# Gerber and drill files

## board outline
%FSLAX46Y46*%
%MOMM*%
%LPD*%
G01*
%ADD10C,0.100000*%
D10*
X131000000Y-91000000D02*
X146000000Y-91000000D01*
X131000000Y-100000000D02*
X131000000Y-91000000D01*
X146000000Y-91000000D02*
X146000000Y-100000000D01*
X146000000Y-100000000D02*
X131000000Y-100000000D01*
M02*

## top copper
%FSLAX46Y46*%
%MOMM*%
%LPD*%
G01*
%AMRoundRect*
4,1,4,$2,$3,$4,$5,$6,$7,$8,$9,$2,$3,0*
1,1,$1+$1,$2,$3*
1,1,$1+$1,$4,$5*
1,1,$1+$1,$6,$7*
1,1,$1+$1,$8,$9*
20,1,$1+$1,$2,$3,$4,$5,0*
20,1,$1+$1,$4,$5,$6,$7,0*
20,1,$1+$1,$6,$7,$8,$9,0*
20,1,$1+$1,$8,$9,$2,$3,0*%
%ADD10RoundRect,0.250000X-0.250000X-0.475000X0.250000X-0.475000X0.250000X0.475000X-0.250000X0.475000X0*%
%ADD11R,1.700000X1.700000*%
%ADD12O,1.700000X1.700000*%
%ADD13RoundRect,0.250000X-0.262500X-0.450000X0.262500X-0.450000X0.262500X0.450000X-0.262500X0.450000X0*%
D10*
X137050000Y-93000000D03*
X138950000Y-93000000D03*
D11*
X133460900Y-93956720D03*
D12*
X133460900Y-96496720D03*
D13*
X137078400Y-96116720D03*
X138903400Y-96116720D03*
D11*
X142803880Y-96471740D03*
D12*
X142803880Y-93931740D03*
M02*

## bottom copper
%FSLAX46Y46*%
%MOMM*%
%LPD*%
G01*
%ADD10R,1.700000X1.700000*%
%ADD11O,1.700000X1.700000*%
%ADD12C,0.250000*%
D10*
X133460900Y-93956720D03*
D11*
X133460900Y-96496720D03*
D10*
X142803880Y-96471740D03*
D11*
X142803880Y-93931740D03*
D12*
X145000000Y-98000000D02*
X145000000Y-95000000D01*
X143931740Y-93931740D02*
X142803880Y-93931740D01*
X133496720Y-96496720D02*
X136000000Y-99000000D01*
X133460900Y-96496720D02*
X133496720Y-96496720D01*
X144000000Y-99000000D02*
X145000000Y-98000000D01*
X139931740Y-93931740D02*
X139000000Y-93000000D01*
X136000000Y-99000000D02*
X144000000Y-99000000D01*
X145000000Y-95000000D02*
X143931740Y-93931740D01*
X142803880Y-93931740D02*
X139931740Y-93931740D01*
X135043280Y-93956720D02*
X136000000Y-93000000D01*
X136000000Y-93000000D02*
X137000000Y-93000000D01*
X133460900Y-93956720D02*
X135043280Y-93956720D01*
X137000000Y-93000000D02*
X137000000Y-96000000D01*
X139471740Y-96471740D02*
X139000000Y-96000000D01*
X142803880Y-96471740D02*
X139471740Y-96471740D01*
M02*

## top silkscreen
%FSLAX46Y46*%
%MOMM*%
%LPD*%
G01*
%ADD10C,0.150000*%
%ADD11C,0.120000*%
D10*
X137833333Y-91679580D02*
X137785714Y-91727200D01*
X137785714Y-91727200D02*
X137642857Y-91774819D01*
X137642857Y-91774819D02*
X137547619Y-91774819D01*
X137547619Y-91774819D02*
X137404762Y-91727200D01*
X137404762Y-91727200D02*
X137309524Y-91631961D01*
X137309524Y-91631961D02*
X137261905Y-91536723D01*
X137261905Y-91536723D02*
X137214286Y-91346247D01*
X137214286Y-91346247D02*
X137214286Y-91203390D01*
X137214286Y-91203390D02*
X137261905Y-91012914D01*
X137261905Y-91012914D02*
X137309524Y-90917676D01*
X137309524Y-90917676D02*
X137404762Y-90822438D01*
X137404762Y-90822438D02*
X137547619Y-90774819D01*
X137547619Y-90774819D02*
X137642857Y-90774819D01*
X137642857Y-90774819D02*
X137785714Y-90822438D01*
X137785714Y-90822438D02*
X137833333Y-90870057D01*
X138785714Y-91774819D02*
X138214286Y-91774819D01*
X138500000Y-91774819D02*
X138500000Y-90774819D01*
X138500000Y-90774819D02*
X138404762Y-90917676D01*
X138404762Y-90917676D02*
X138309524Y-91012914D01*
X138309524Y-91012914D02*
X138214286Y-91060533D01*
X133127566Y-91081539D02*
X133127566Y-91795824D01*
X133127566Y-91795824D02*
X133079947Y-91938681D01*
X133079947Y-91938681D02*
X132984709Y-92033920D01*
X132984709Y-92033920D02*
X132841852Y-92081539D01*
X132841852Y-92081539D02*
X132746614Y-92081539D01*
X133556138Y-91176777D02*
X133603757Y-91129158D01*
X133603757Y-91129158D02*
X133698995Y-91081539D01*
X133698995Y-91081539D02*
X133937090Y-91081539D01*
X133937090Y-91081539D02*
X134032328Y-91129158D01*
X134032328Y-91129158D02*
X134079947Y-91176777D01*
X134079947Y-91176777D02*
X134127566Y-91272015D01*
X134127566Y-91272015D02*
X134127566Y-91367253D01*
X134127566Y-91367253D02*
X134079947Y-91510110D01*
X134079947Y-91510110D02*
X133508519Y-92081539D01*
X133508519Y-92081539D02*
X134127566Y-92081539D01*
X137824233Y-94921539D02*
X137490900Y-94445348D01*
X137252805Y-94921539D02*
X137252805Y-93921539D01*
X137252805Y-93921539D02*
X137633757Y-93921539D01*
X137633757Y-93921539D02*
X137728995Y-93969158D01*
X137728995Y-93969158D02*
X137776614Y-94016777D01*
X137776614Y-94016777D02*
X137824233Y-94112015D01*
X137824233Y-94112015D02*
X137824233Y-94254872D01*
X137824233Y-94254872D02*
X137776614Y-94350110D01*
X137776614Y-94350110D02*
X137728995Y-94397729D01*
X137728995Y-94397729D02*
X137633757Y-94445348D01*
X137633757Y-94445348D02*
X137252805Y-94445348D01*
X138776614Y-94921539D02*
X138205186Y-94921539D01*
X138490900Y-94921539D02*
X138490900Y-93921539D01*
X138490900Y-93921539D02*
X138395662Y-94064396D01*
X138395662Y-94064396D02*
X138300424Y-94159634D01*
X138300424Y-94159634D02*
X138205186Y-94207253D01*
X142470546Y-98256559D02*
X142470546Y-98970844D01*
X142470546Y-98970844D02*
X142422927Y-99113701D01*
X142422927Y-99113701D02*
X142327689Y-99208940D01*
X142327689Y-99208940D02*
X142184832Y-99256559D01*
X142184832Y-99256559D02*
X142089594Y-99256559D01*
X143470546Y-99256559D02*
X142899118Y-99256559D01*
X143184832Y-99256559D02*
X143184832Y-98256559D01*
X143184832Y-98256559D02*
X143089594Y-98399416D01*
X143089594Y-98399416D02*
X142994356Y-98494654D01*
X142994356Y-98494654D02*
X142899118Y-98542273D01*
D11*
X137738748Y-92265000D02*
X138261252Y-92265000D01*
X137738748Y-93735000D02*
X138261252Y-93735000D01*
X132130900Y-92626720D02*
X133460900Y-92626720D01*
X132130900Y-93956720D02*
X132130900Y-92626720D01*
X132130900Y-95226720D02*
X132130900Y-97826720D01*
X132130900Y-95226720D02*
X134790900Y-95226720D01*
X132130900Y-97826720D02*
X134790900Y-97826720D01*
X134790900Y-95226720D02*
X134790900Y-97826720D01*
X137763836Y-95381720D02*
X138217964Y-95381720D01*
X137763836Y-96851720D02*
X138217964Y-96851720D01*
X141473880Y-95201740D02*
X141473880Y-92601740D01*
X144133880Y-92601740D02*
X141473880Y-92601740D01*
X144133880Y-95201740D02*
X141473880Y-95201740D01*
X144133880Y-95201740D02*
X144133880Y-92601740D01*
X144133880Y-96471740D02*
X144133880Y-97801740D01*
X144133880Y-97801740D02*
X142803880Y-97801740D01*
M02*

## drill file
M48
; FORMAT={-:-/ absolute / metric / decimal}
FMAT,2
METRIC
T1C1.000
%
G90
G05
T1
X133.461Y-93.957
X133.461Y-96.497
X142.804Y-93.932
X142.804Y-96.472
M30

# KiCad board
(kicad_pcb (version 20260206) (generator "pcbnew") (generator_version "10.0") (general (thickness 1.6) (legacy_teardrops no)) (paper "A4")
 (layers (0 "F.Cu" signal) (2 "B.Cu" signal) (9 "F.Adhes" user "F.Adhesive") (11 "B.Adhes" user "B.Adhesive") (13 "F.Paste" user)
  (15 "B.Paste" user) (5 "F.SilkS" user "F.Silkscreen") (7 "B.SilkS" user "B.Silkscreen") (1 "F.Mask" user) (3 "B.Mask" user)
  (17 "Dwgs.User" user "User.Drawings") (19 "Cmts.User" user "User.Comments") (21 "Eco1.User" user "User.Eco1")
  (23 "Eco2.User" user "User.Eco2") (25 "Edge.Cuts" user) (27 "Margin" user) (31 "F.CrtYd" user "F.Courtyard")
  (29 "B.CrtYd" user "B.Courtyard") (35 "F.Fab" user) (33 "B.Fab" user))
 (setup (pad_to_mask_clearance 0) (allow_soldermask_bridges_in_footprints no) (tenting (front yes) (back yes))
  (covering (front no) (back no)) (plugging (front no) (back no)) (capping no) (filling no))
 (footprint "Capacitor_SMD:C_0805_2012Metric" (layer "F.Cu") (at 138 93)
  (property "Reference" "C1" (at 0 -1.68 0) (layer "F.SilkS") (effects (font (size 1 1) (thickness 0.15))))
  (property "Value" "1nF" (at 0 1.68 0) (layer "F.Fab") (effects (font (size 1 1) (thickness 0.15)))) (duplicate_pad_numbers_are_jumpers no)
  (fp_line (start -0.261252 -0.735) (end 0.261252 -0.735) (stroke (width 0.12) (type solid)) (layer "F.SilkS"))
  (fp_line (start -0.261252 0.735) (end 0.261252 0.735) (stroke (width 0.12) (type solid)) (layer "F.SilkS"))
  (pad "1" smd roundrect (at -0.95 0) (size 1 1.45) (layers "F.Cu" "F.Mask" "F.Paste") (roundrect_rratio 0.25) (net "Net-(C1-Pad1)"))
  (pad "2" smd roundrect (at 0.95 0) (size 1 1.45) (layers "F.Cu" "F.Mask" "F.Paste") (roundrect_rratio 0.25) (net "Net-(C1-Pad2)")))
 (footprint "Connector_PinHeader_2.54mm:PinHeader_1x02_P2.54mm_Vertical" (layer "F.Cu") (at 133.4609 93.95672)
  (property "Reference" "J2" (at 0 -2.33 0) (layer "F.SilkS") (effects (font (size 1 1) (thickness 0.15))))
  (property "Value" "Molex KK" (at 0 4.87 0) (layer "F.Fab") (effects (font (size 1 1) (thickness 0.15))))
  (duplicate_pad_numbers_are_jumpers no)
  (fp_line (start -1.33 -1.33) (end 0 -1.33) (stroke (width 0.12) (type solid)) (layer "F.SilkS"))
  (fp_line (start -1.33 0) (end -1.33 -1.33) (stroke (width 0.12) (type solid)) (layer "F.SilkS"))
  (fp_line (start -1.33 1.27) (end -1.33 3.87) (stroke (width 0.12) (type solid)) (layer "F.SilkS"))
  (fp_line (start -1.33 1.27) (end 1.33 1.27) (stroke (width 0.12) (type solid)) (layer "F.SilkS"))
  (fp_line (start -1.33 3.87) (end 1.33 3.87) (stroke (width 0.12) (type solid)) (layer "F.SilkS"))
  (fp_line (start 1.33 1.27) (end 1.33 3.87) (stroke (width 0.12) (type solid)) (layer "F.SilkS"))
  (pad "1" thru_hole rect (at 0 0) (size 1.7 1.7) (drill 1) (layers "*.Cu" "*.Mask") (remove_unused_layers no) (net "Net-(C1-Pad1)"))
  (pad "2" thru_hole oval (at 0 2.54) (size 1.7 1.7) (drill 1) (layers "*.Cu" "*.Mask") (remove_unused_layers no) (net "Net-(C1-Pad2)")))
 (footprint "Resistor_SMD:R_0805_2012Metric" (layer "F.Cu") (at 137.9909 96.11672)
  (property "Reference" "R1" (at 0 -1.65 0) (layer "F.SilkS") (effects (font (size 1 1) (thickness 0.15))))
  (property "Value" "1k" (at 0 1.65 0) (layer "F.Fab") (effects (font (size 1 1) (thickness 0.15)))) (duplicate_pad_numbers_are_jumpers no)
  (fp_line (start -0.227064 -0.735) (end 0.227064 -0.735) (stroke (width 0.12) (type solid)) (layer "F.SilkS"))
  (fp_line (start -0.227064 0.735) (end 0.227064 0.735) (stroke (width 0.12) (type solid)) (layer "F.SilkS"))
  (pad "1" smd roundrect (at -0.9125 0) (size 1.025 1.4) (layers "F.Cu" "F.Mask" "F.Paste") (roundrect_rratio 0.243902)
   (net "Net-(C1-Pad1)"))
  (pad "2" smd roundrect (at 0.9125 0) (size 1.025 1.4) (layers "F.Cu" "F.Mask" "F.Paste") (roundrect_rratio 0.243902) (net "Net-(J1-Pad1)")))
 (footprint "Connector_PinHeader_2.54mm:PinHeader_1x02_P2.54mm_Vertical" (layer "F.Cu") (at 142.80388 96.47174 180)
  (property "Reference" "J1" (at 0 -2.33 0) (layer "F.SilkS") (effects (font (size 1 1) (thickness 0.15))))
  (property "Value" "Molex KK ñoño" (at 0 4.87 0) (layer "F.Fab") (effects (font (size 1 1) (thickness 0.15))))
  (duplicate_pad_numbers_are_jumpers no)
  (fp_line (start 1.33 1.27) (end 1.33 3.87) (stroke (width 0.12) (type solid)) (layer "F.SilkS"))
  (fp_line (start -1.33 3.87) (end 1.33 3.87) (stroke (width 0.12) (type solid)) (layer "F.SilkS"))
  (fp_line (start -1.33 1.27) (end 1.33 1.27) (stroke (width 0.12) (type solid)) (layer "F.SilkS"))
  (fp_line (start -1.33 1.27) (end -1.33 3.87) (stroke (width 0.12) (type solid)) (layer "F.SilkS"))
  (fp_line (start -1.33 0) (end -1.33 -1.33) (stroke (width 0.12) (type solid)) (layer "F.SilkS"))
  (fp_line (start -1.33 -1.33) (end 0 -1.33) (stroke (width 0.12) (type solid)) (layer "F.SilkS"))
  (pad "1" thru_hole rect (at 0 0 180) (size 1.7 1.7) (drill 1) (layers "*.Cu" "*.Mask") (remove_unused_layers no) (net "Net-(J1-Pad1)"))
  (pad "2" thru_hole oval (at 0 2.54 180) (size 1.7 1.7) (drill 1) (layers "*.Cu" "*.Mask") (remove_unused_layers no) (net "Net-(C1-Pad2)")))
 (gr_line (start 131 91) (end 146 91) (stroke (width 0.1) (type solid)) (layer "Edge.Cuts"))
 (gr_line (start 131 100) (end 131 91) (stroke (width 0.1) (type solid)) (layer "Edge.Cuts"))
 (gr_line (start 146 91) (end 146 100) (stroke (width 0.1) (type solid)) (layer "Edge.Cuts"))
 (gr_line (start 146 100) (end 131 100) (stroke (width 0.1) (type solid)) (layer "Edge.Cuts"))
 (segment (start 145 98) (end 145 95) (width 0.25) (layer "B.Cu") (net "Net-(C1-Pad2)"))
 (segment (start 143.93174 93.93174) (end 142.80388 93.93174) (width 0.25) (layer "B.Cu") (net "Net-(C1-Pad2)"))
 (segment (start 133.49672 96.49672) (end 136 99) (width 0.25) (layer "B.Cu") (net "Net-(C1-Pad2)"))
 (segment (start 133.4609 96.49672) (end 133.49672 96.49672) (width 0.25) (layer "B.Cu") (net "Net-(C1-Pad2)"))
 (segment (start 144 99) (end 145 98) (width 0.25) (layer "B.Cu") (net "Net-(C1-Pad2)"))
 (segment (start 139.93174 93.93174) (end 139 93) (width 0.25) (layer "B.Cu") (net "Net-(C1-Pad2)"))
 (segment (start 136 99) (end 144 99) (width 0.25) (layer "B.Cu") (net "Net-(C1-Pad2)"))
 (segment (start 145 95) (end 143.93174 93.93174) (width 0.25) (layer "B.Cu") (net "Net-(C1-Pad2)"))
 (segment (start 142.80388 93.93174) (end 139.93174 93.93174) (width 0.25) (layer "B.Cu") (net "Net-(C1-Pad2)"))
 (segment (start 135.04328 93.95672) (end 136 93) (width 0.25) (layer "B.Cu") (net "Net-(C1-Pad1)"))
 (segment (start 136 93) (end 137 93) (width 0.25) (layer "B.Cu") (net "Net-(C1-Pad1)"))
 (segment (start 133.4609 93.95672) (end 135.04328 93.95672) (width 0.25) (layer "B.Cu") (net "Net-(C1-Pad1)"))
 (segment (start 137 93) (end 137 96) (width 0.25) (layer "B.Cu") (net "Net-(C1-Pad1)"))
 (segment (start 139.47174 96.47174) (end 139 96) (width 0.25) (layer "B.Cu") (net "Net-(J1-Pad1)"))
 (segment (start 142.80388 96.47174) (end 139.47174 96.47174) (width 0.25) (layer "B.Cu") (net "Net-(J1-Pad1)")))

